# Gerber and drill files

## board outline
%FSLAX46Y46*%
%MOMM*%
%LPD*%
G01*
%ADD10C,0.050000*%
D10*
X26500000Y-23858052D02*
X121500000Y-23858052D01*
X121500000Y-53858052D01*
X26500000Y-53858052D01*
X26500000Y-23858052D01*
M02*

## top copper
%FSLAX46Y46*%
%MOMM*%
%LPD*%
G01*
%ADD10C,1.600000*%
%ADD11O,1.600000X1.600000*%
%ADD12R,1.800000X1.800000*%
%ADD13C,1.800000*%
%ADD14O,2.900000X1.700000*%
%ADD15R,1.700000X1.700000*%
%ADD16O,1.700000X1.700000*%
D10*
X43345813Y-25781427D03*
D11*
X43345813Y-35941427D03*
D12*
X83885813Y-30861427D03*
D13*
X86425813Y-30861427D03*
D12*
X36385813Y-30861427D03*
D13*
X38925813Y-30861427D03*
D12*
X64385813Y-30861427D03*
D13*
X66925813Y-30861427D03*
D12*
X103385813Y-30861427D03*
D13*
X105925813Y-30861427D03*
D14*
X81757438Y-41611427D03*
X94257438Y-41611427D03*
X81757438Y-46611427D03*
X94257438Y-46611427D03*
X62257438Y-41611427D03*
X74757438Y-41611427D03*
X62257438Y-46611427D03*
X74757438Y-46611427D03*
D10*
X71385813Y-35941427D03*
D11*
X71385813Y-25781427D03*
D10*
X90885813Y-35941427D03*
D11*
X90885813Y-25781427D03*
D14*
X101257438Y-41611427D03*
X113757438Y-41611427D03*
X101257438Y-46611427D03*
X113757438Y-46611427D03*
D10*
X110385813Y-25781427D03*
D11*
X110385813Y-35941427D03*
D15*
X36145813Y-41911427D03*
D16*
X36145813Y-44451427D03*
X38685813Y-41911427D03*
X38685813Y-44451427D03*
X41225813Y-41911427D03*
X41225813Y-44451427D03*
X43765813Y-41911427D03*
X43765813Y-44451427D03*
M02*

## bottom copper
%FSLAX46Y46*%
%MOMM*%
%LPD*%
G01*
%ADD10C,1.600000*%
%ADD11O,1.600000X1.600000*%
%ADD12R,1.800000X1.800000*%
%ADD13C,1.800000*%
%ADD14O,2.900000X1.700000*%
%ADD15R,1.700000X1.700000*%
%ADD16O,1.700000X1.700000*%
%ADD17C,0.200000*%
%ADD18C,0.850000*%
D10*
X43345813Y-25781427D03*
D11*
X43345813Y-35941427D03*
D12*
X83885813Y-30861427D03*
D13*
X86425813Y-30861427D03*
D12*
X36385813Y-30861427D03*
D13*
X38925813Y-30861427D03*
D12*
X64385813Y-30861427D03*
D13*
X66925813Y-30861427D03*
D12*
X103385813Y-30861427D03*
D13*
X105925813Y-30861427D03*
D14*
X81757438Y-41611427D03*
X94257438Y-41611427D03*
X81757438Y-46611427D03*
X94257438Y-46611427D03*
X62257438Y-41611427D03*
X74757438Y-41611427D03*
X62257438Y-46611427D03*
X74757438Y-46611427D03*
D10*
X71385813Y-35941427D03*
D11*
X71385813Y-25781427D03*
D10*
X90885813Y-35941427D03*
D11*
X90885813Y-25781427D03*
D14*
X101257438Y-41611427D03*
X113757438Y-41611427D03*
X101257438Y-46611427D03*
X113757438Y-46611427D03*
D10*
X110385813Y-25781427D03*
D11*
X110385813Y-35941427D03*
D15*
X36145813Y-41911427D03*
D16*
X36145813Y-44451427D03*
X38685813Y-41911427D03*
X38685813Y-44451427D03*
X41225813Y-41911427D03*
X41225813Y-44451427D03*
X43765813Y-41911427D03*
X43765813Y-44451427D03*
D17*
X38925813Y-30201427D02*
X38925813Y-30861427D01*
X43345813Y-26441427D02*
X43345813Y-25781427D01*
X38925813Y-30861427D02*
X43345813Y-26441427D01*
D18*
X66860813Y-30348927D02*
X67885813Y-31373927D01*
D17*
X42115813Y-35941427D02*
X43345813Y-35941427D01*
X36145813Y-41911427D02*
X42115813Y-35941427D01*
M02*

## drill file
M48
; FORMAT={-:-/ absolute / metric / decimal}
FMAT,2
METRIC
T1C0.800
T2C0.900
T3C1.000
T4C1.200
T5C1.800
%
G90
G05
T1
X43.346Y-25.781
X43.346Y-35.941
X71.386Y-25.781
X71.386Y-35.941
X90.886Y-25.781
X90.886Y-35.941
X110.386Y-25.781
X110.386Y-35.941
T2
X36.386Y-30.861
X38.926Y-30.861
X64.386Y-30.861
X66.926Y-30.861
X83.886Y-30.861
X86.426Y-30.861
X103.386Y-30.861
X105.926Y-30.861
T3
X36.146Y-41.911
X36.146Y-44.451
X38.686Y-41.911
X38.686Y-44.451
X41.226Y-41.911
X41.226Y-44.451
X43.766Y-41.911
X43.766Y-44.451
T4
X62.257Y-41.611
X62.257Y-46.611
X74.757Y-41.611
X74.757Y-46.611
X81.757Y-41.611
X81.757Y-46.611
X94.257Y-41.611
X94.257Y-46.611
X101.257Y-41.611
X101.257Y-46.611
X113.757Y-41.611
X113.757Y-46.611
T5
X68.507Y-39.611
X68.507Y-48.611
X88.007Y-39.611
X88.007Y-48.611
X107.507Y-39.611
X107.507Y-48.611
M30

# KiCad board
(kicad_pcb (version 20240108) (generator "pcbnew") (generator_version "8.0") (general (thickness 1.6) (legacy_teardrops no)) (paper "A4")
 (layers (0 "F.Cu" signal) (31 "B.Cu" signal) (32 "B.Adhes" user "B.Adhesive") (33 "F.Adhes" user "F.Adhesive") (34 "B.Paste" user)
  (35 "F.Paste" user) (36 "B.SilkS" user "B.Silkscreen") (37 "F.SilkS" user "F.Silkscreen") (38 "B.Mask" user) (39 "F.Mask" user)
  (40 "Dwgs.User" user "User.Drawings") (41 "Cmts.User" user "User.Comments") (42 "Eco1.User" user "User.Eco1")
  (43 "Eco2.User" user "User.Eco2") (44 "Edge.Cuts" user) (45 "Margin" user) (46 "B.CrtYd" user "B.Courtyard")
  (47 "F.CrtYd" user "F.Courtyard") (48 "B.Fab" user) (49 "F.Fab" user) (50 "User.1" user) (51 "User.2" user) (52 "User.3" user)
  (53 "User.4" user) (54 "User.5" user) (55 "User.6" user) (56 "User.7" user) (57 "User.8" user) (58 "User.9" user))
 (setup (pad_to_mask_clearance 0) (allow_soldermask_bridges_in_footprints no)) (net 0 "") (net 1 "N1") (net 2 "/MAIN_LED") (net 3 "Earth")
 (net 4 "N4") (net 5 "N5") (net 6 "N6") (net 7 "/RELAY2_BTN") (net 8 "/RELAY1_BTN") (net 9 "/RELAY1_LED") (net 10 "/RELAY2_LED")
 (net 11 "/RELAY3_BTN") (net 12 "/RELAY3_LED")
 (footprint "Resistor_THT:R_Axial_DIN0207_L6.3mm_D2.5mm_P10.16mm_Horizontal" (layer "F.Cu") (at 43.345813 25.781427 -90)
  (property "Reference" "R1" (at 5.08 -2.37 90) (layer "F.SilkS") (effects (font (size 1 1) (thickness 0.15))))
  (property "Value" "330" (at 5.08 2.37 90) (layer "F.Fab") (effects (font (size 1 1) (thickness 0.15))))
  (pad "1" thru_hole circle (at 0 0 270) (size 1.6 1.6) (drill 0.8) (layers "*.Cu" "*.Mask") (remove_unused_layers no) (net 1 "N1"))
  (pad "2" thru_hole oval (at 10.16 0 270) (size 1.6 1.6) (drill 0.8) (layers "*.Cu" "*.Mask") (remove_unused_layers no) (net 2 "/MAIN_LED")))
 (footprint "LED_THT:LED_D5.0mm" (layer "F.Cu") (at 83.885813 30.861427)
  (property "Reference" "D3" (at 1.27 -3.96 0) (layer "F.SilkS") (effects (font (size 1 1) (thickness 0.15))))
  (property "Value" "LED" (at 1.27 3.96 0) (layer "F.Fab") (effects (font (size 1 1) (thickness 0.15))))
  (pad "1" thru_hole rect (at 0 0) (size 1.8 1.8) (drill 0.9) (layers "*.Cu" "*.Mask") (remove_unused_layers no) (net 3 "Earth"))
  (pad "2" thru_hole circle (at 2.54 0) (size 1.8 1.8) (drill 0.9) (layers "*.Cu" "*.Mask") (remove_unused_layers no) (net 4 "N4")))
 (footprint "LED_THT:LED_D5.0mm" (layer "F.Cu") (at 36.385813 30.861427)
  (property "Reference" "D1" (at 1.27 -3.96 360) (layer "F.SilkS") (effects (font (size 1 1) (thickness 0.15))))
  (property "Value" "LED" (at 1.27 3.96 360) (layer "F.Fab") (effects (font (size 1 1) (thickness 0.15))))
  (pad "1" thru_hole rect (at 0 0) (size 1.8 1.8) (drill 0.9) (layers "*.Cu" "*.Mask") (remove_unused_layers no) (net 3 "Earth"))
  (pad "2" thru_hole circle (at 2.54 0) (size 1.8 1.8) (drill 0.9) (layers "*.Cu" "*.Mask") (remove_unused_layers no) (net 1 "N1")))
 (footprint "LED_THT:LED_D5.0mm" (layer "F.Cu") (at 64.385813 30.861427)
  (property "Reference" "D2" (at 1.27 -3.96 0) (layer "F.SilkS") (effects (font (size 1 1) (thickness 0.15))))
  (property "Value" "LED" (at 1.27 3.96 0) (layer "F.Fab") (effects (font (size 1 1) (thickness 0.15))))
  (pad "1" thru_hole rect (at 0 0) (size 1.8 1.8) (drill 0.9) (layers "*.Cu" "*.Mask") (remove_unused_layers no) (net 3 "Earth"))
  (pad "2" thru_hole circle (at 2.54 0) (size 1.8 1.8) (drill 0.9) (layers "*.Cu" "*.Mask") (remove_unused_layers no) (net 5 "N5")))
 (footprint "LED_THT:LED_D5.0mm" (layer "F.Cu") (at 103.385813 30.861427)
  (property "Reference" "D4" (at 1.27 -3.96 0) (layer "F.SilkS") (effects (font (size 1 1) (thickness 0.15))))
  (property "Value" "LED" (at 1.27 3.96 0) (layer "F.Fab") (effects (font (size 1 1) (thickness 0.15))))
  (pad "1" thru_hole rect (at 0 0) (size 1.8 1.8) (drill 0.9) (layers "*.Cu" "*.Mask") (remove_unused_layers no) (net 3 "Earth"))
  (pad "2" thru_hole circle (at 2.54 0) (size 1.8 1.8) (drill 0.9) (layers "*.Cu" "*.Mask") (remove_unused_layers no) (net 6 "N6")))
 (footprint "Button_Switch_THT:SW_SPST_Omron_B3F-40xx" (layer "F.Cu") (at 81.757438 41.611427)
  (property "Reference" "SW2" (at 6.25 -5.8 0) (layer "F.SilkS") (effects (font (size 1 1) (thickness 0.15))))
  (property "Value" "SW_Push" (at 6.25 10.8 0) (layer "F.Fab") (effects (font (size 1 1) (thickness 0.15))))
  (pad "" np_thru_hole circle (at 6.25 -2) (size 1.8 1.8) (drill 1.8) (layers "F&B.Cu" "*.Mask"))
  (pad "" np_thru_hole circle (at 6.25 7) (size 1.8 1.8) (drill 1.8) (layers "F&B.Cu" "*.Mask"))
  (pad "1" thru_hole oval (at 0 0) (size 2.9 1.7) (drill 1.2) (layers "*.Cu" "*.Mask") (remove_unused_layers no) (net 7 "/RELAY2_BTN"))
  (pad "1" thru_hole oval (at 12.5 0) (size 2.9 1.7) (drill 1.2) (layers "*.Cu" "*.Mask") (remove_unused_layers no) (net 7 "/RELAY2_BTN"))
  (pad "2" thru_hole oval (at 0 5) (size 2.9 1.7) (drill 1.2) (layers "*.Cu" "*.Mask") (remove_unused_layers no) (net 3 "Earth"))
  (pad "2" thru_hole oval (at 12.5 5) (size 2.9 1.7) (drill 1.2) (layers "*.Cu" "*.Mask") (remove_unused_layers no) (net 3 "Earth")))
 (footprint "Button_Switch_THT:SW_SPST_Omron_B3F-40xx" (layer "F.Cu") (at 62.257438 41.611427)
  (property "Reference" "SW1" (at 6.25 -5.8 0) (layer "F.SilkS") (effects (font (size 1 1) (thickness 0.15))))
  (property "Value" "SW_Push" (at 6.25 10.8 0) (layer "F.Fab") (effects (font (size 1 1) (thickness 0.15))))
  (pad "" np_thru_hole circle (at 6.25 -2) (size 1.8 1.8) (drill 1.8) (layers "F&B.Cu" "*.Mask"))
  (pad "" np_thru_hole circle (at 6.25 7) (size 1.8 1.8) (drill 1.8) (layers "F&B.Cu" "*.Mask"))
  (pad "1" thru_hole oval (at 0 0) (size 2.9 1.7) (drill 1.2) (layers "*.Cu" "*.Mask") (remove_unused_layers no) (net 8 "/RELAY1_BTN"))
  (pad "1" thru_hole oval (at 12.5 0) (size 2.9 1.7) (drill 1.2) (layers "*.Cu" "*.Mask") (remove_unused_layers no) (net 8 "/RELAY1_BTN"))
  (pad "2" thru_hole oval (at 0 5) (size 2.9 1.7) (drill 1.2) (layers "*.Cu" "*.Mask") (remove_unused_layers no) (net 3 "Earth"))
  (pad "2" thru_hole oval (at 12.5 5) (size 2.9 1.7) (drill 1.2) (layers "*.Cu" "*.Mask") (remove_unused_layers no) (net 3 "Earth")))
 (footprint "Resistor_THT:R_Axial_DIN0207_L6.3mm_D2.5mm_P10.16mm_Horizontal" (layer "F.Cu") (at 71.385813 35.941427 90)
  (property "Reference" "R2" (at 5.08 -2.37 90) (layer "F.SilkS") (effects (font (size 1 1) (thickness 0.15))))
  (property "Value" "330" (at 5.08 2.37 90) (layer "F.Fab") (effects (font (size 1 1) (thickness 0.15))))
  (pad "1" thru_hole circle (at 0 0 90) (size 1.6 1.6) (drill 0.8) (layers "*.Cu" "*.Mask") (remove_unused_layers no) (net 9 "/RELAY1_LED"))
  (pad "2" thru_hole oval (at 10.16 0 90) (size 1.6 1.6) (drill 0.8) (layers "*.Cu" "*.Mask") (remove_unused_layers no) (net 5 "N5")))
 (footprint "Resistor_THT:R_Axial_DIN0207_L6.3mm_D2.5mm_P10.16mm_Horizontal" (layer "F.Cu") (at 90.885813 35.941427 90)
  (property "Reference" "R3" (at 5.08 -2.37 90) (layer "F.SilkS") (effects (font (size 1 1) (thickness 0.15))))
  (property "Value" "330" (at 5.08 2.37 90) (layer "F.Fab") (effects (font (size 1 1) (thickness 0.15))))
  (pad "1" thru_hole circle (at 0 0 90) (size 1.6 1.6) (drill 0.8) (layers "*.Cu" "*.Mask") (remove_unused_layers no) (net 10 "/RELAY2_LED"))
  (pad "2" thru_hole oval (at 10.16 0 90) (size 1.6 1.6) (drill 0.8) (layers "*.Cu" "*.Mask") (remove_unused_layers no) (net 4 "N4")))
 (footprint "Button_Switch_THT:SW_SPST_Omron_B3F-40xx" (layer "F.Cu") (at 101.257438 41.611427)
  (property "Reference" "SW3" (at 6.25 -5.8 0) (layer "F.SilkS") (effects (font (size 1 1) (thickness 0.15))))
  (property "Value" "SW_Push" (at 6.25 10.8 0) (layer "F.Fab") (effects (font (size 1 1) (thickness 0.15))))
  (pad "" np_thru_hole circle (at 6.25 -2) (size 1.8 1.8) (drill 1.8) (layers "F&B.Cu" "*.Mask"))
  (pad "" np_thru_hole circle (at 6.25 7) (size 1.8 1.8) (drill 1.8) (layers "F&B.Cu" "*.Mask"))
  (pad "1" thru_hole oval (at 0 0) (size 2.9 1.7) (drill 1.2) (layers "*.Cu" "*.Mask") (remove_unused_layers no) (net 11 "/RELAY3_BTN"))
  (pad "1" thru_hole oval (at 12.5 0) (size 2.9 1.7) (drill 1.2) (layers "*.Cu" "*.Mask") (remove_unused_layers no) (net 11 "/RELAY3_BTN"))
  (pad "2" thru_hole oval (at 0 5) (size 2.9 1.7) (drill 1.2) (layers "*.Cu" "*.Mask") (remove_unused_layers no) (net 3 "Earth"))
  (pad "2" thru_hole oval (at 12.5 5) (size 2.9 1.7) (drill 1.2) (layers "*.Cu" "*.Mask") (remove_unused_layers no) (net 3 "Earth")))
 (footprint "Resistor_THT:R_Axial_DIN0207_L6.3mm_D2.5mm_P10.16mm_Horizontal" (layer "F.Cu") (at 110.385813 25.781427 -90)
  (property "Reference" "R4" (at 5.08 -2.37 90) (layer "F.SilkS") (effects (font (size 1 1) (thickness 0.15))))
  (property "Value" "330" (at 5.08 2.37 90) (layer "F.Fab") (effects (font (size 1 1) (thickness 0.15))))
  (pad "1" thru_hole circle (at 0 0 270) (size 1.6 1.6) (drill 0.8) (layers "*.Cu" "*.Mask") (remove_unused_layers no) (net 6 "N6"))
  (pad "2" thru_hole oval (at 10.16 0 270) (size 1.6 1.6) (drill 0.8) (layers "*.Cu" "*.Mask") (remove_unused_layers no)
   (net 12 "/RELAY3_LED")))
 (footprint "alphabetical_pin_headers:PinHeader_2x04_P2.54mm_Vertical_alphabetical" (layer "B.Cu") (at 36.145813 41.911427 -90)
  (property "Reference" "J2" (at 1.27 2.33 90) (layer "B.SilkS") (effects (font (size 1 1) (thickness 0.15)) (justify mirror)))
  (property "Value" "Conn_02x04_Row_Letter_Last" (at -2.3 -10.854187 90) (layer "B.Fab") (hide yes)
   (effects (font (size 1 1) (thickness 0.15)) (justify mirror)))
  (pad "1a" thru_hole rect (at 0 0 270) (size 1.7 1.7) (drill 1) (layers "*.Cu" "*.Mask") (remove_unused_layers no) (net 2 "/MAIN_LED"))
  (pad "1b" thru_hole oval (at 2.54 0 270) (size 1.7 1.7) (drill 1) (layers "*.Cu" "*.Mask") (remove_unused_layers no) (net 3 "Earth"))
  (pad "2a" thru_hole oval (at 0 -2.54 270) (size 1.7 1.7) (drill 1) (layers "*.Cu" "*.Mask") (remove_unused_layers no)
   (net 9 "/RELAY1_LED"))
  (pad "2b" thru_hole oval (at 2.54 -2.54 270) (size 1.7 1.7) (drill 1) (layers "*.Cu" "*.Mask") (remove_unused_layers no)
   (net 8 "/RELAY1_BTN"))
  (pad "3a" thru_hole oval (at 0 -5.08 270) (size 1.7 1.7) (drill 1) (layers "*.Cu" "*.Mask") (remove_unused_layers no)
   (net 10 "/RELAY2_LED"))
  (pad "3b" thru_hole oval (at 2.54 -5.08 270) (size 1.7 1.7) (drill 1) (layers "*.Cu" "*.Mask") (remove_unused_layers no)
   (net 7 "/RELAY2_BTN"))
  (pad "4a" thru_hole oval (at 0 -7.62 270) (size 1.7 1.7) (drill 1) (layers "*.Cu" "*.Mask") (remove_unused_layers no)
   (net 12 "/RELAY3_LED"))
  (pad "4b" thru_hole oval (at 2.54 -7.62 270) (size 1.7 1.7) (drill 1) (layers "*.Cu" "*.Mask") (remove_unused_layers no)
   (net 11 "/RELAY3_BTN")))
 (gr_rect (start 26.5 23.858052) (end 121.5 53.858052) (stroke (width 0.05) (type default)) (fill none) (layer "Edge.Cuts"))
 (segment (start 38.925813 30.201427) (end 38.925813 30.861427) (width 0.2) (layer "B.Cu") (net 1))
 (segment (start 43.345813 26.441427) (end 43.345813 25.781427) (width 0.2) (layer "B.Cu") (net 1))
 (segment (start 38.925813 30.861427) (end 43.345813 26.441427) (width 0.2) (layer "B.Cu") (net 1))
 (segment (start 66.860813 30.348927) (end 67.885813 31.373927) (width 0.85) (layer "B.Cu") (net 5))
 (segment (start 42.115813 35.941427) (end 43.345813 35.941427) (width 0.2) (layer "B.Cu") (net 2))
 (segment (start 36.145813 41.911427) (end 42.115813 35.941427) (width 0.2) (layer "B.Cu") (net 2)))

